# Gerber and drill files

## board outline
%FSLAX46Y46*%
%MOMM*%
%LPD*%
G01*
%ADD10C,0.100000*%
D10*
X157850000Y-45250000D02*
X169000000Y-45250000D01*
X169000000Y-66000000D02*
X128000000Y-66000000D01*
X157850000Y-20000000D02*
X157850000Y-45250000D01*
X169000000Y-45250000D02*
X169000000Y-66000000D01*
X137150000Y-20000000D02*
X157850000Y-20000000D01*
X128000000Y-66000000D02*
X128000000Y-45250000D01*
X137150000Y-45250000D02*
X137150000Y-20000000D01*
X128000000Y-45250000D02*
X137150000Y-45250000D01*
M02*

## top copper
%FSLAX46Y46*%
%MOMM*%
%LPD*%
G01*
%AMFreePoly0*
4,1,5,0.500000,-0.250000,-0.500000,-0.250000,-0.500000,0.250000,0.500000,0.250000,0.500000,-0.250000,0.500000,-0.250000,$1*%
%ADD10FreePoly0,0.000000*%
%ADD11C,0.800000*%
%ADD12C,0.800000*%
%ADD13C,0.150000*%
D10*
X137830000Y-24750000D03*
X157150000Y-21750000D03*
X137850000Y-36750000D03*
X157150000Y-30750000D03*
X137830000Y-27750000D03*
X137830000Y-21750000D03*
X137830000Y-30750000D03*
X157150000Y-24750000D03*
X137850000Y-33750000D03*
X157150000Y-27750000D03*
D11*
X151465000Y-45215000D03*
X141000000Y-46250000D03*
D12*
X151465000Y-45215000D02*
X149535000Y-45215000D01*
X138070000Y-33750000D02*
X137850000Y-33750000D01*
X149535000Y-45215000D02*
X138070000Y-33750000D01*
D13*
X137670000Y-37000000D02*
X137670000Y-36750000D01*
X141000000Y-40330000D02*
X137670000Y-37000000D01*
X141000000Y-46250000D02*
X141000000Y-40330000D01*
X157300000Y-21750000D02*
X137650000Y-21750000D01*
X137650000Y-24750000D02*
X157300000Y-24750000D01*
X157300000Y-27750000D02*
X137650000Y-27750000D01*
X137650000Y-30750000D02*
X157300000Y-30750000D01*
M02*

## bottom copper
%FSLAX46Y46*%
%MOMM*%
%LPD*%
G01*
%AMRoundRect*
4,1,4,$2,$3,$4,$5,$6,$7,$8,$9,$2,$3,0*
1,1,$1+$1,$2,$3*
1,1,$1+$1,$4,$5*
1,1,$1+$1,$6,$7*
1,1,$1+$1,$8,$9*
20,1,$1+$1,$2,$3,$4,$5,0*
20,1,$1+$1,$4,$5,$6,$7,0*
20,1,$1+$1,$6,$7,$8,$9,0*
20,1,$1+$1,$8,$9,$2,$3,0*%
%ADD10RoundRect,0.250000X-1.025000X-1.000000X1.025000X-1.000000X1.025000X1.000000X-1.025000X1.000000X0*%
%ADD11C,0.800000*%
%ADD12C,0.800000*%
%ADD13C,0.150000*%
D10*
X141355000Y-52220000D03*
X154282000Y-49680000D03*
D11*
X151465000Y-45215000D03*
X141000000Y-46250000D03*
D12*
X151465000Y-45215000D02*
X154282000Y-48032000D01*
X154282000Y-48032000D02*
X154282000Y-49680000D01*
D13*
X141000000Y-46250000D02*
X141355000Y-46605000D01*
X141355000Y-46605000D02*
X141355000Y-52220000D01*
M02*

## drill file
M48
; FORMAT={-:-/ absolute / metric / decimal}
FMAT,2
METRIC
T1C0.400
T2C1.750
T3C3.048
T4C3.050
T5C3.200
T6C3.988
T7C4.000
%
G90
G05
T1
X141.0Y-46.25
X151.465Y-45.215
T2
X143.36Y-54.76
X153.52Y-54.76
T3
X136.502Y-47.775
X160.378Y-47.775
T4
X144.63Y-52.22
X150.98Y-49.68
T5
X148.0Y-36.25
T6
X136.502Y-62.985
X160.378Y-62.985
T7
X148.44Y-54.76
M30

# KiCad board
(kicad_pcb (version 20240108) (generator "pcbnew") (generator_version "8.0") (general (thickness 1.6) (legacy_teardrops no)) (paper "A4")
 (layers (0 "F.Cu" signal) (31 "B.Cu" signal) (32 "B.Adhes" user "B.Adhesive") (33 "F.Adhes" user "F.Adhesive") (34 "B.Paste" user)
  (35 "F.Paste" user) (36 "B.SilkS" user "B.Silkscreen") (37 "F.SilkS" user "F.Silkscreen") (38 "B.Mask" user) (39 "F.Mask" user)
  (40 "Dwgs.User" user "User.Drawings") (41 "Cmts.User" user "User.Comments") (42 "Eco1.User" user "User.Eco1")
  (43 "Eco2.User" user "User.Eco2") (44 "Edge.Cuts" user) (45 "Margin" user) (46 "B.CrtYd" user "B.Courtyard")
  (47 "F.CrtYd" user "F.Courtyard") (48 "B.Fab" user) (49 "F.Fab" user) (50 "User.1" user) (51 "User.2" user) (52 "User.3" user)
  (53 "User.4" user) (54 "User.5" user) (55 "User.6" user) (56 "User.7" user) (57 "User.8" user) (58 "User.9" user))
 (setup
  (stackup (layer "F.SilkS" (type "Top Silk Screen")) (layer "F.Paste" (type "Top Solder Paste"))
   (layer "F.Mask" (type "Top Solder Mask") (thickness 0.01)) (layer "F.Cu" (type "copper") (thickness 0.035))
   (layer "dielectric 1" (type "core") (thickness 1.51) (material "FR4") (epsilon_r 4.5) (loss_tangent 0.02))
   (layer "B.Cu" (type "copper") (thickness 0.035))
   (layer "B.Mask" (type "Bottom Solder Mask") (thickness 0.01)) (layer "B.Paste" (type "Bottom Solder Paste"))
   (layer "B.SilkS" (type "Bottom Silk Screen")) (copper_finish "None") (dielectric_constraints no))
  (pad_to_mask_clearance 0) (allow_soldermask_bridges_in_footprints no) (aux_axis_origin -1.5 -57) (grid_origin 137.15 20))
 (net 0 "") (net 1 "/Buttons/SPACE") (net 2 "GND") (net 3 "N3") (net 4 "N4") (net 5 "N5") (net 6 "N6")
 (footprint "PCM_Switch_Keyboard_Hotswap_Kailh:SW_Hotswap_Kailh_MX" (layer "F.Cu") (at 148.44 54.76)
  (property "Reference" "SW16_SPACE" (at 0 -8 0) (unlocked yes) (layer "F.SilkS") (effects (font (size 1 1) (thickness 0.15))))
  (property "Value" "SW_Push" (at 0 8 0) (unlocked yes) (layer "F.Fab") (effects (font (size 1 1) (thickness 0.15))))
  (pad "" np_thru_hole circle (at -5.08 0) (size 1.75 1.75) (drill 1.75) (layers "*.Cu" "*.Mask"))
  (pad "" np_thru_hole circle (at -3.81 -2.54) (size 3.05 3.05) (drill 3.05) (layers "*.Cu" "*.Mask"))
  (pad "" np_thru_hole circle (at 0 0) (size 4 4) (drill 4) (layers "*.Cu" "*.Mask"))
  (pad "" np_thru_hole circle (at 2.54 -5.08) (size 3.05 3.05) (drill 3.05) (layers "*.Cu" "*.Mask"))
  (pad "" np_thru_hole circle (at 5.08 0) (size 1.75 1.75) (drill 1.75) (layers "*.Cu" "*.Mask"))
  (pad "1" smd roundrect (at -7.085 -2.54) (size 2.55 2.5) (layers "B.Cu" "B.Paste" "B.Mask") (roundrect_rratio 0.1)
   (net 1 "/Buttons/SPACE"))
  (pad "2" smd roundrect (at 5.842 -5.08) (size 2.55 2.5) (layers "B.Cu" "B.Paste" "B.Mask") (roundrect_rratio 0.1) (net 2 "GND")))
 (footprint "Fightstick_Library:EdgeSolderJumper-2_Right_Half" (layer "F.Cu") (at 137.18 24.75)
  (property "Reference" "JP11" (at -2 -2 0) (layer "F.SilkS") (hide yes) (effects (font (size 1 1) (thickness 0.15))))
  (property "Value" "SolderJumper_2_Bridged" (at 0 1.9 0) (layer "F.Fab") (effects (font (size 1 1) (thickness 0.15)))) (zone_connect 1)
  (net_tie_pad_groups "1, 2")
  (pad "2" smd custom (at 0.65 0) (size 1 0.5) (layers "F.Cu" "F.Mask") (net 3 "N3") (zone_connect 2) (thermal_bridge_angle 45)
   (options (clearance outline) (anchor rect)) (primitives)))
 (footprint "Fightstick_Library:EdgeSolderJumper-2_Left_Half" (layer "F.Cu") (at 157.8 21.75)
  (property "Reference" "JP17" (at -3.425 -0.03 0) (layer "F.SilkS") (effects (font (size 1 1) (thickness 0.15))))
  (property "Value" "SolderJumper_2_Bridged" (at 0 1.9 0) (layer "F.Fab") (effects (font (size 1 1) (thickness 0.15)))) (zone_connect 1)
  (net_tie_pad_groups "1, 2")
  (pad "1" smd custom (at -0.65 0) (size 1 0.5) (layers "F.Cu" "F.Mask") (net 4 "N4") (zone_connect 2) (thermal_bridge_angle 45)
   (options (clearance outline) (anchor rect)) (primitives)))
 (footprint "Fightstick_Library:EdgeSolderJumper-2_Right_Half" (layer "F.Cu") (at 137.2 36.75)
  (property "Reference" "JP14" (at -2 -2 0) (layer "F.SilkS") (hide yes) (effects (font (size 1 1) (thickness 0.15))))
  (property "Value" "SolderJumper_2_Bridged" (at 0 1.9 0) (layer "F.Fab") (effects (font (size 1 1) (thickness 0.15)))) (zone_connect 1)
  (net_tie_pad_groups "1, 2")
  (pad "2" smd custom (at 0.65 0) (size 1 0.5) (layers "F.Cu" "F.Mask") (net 1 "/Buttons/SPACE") (zone_connect 2) (thermal_bridge_angle 45)
   (options (clearance outline) (anchor rect)) (primitives)))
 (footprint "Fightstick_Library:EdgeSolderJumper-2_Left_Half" (layer "F.Cu") (at 157.8 30.75)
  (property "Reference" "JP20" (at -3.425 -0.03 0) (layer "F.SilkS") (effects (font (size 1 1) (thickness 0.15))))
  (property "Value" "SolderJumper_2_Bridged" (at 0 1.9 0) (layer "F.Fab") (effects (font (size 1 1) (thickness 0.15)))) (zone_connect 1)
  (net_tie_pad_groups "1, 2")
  (pad "1" smd custom (at -0.65 0) (size 1 0.5) (layers "F.Cu" "F.Mask") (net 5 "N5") (zone_connect 2) (thermal_bridge_angle 45)
   (options (clearance outline) (anchor rect)) (primitives)))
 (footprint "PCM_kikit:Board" (layer "F.Cu") (at 128 56.75)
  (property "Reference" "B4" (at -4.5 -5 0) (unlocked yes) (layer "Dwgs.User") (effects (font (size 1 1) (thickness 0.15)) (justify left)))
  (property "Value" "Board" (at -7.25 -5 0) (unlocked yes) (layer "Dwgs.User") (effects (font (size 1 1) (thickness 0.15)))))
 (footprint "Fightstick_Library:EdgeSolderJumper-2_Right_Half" (layer "F.Cu") (at 137.18 27.75)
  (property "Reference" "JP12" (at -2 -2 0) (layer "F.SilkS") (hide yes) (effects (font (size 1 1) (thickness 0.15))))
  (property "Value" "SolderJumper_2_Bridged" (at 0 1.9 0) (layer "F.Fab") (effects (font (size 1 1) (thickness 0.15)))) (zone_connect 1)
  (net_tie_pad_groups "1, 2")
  (pad "2" smd custom (at 0.65 0) (size 1 0.5) (layers "F.Cu" "F.Mask") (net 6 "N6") (zone_connect 2) (thermal_bridge_angle 45)
   (options (clearance outline) (anchor rect)) (primitives)))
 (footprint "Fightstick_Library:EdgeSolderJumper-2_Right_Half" (layer "F.Cu") (at 137.18 21.75)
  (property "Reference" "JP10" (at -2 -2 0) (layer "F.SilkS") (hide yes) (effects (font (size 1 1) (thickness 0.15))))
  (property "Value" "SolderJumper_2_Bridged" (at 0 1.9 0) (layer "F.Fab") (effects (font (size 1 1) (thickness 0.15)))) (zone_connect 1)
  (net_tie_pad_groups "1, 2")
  (pad "2" smd custom (at 0.65 0) (size 1 0.5) (layers "F.Cu" "F.Mask") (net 4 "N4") (zone_connect 2) (thermal_bridge_angle 45)
   (options (clearance outline) (anchor rect)) (primitives)))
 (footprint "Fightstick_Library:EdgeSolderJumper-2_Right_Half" (layer "F.Cu") (at 137.18 30.75)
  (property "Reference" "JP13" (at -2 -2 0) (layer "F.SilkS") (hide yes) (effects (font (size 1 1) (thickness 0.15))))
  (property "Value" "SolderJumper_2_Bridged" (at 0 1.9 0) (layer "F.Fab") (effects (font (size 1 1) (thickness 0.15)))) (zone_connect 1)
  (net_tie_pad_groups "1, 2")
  (pad "2" smd custom (at 0.65 0) (size 1 0.5) (layers "F.Cu" "F.Mask") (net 5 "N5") (zone_connect 2) (thermal_bridge_angle 45)
   (options (clearance outline) (anchor rect)) (primitives)))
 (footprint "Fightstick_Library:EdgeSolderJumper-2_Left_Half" (layer "F.Cu") (at 157.8 24.75)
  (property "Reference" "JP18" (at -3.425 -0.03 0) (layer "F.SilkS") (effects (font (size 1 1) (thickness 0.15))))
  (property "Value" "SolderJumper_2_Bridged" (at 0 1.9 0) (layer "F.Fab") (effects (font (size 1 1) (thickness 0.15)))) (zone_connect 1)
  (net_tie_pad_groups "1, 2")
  (pad "1" smd custom (at -0.65 0) (size 1 0.5) (layers "F.Cu" "F.Mask") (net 3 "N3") (zone_connect 2) (thermal_bridge_angle 45)
   (options (clearance outline) (anchor rect)) (primitives)))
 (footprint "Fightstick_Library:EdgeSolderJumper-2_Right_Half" (layer "F.Cu") (at 137.2 33.75)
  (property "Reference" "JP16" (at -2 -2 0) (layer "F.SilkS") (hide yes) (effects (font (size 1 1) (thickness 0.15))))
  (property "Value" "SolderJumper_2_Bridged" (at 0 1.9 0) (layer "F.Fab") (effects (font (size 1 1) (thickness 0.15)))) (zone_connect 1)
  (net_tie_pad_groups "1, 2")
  (pad "2" smd custom (at 0.65 0) (size 1 0.5) (layers "F.Cu" "F.Mask") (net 2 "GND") (zone_connect 2) (thermal_bridge_angle 45)
   (options (clearance outline) (anchor rect)) (primitives)))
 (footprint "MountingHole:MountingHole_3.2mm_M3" (layer "F.Cu") (at 148 36.25)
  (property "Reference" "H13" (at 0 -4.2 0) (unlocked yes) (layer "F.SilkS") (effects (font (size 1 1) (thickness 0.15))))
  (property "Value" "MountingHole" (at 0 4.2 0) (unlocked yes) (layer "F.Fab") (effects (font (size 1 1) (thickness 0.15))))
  (pad "" np_thru_hole circle (at 0 0) (size 3.2 3.2) (drill 3.2) (layers "*.Cu" "*.Mask")))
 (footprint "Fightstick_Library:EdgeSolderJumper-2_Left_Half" (layer "F.Cu") (at 157.8 27.75)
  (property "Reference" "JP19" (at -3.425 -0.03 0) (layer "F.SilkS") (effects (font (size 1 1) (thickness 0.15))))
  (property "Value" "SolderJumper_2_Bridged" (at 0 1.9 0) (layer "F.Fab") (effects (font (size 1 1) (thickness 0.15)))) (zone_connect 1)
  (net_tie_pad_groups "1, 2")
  (pad "1" smd custom (at -0.65 0) (size 1 0.5) (layers "F.Cu" "F.Mask") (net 6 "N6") (zone_connect 2) (thermal_bridge_angle 45)
   (options (clearance outline) (anchor rect)) (primitives)))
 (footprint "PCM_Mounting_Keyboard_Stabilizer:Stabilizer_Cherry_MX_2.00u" (layer "F.Cu") (at 148.44 54.76)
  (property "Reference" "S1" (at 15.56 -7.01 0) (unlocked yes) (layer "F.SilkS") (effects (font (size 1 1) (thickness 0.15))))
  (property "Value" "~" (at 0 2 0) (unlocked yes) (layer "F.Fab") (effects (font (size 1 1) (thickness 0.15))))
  (pad "" np_thru_hole circle (at -11.938 -6.985) (size 3.048 3.048) (drill 3.048) (layers "*.Cu" "*.Mask"))
  (pad "" np_thru_hole circle (at -11.938 8.225) (size 3.9878 3.9878) (drill 3.9878) (layers "*.Cu" "*.Mask"))
  (pad "" np_thru_hole circle (at 11.938 -6.985) (size 3.048 3.048) (drill 3.048) (layers "*.Cu" "*.Mask"))
  (pad "" np_thru_hole circle (at 11.938 8.225) (size 3.9878 3.9878) (drill 3.9878) (layers "*.Cu" "*.Mask")))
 (gr_line (start 157.85 45.25) (end 169 45.25) (stroke (width 0.1) (type default)) (layer "Edge.Cuts"))
 (gr_line (start 169 66) (end 128 66) (stroke (width 0.1) (type default)) (layer "Edge.Cuts"))
 (gr_line (start 157.85 20) (end 157.85 45.25) (stroke (width 0.1) (type default)) (layer "Edge.Cuts"))
 (gr_line (start 169 45.25) (end 169 66) (stroke (width 0.1) (type default)) (layer "Edge.Cuts"))
 (gr_line (start 137.15 20) (end 157.85 20) (stroke (width 0.1) (type default)) (layer "Edge.Cuts"))
 (gr_line (start 128 66) (end 128 45.25) (stroke (width 0.1) (type default)) (layer "Edge.Cuts"))
 (gr_line (start 137.15 45.25) (end 137.15 20) (stroke (width 0.1) (type default)) (layer "Edge.Cuts"))
 (gr_line (start 128 45.25) (end 137.15 45.25) (stroke (width 0.1) (type default)) (layer "Edge.Cuts"))
 (segment (start 151.465 45.215) (end 149.535 45.215) (width 0.8) (layer "F.Cu") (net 2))
 (segment (start 138.07 33.75) (end 137.85 33.75) (width 0.8) (layer "F.Cu") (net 2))
 (segment (start 149.535 45.215) (end 138.07 33.75) (width 0.8) (layer "F.Cu") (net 2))
 (via (at 151.465 45.215) (size 0.8) (drill 0.4) (layers "F.Cu" "B.Cu") (free yes) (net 2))
 (segment (start 151.465 45.215) (end 154.282 48.032) (width 0.8) (layer "B.Cu") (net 2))
 (segment (start 154.282 48.032) (end 154.282 49.68) (width 0.8) (layer "B.Cu") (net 2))
 (segment (start 137.67 37) (end 137.67 36.75) (width 0.15) (layer "F.Cu") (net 1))
 (segment (start 141 40.33) (end 137.67 37) (width 0.15) (layer "F.Cu") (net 1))
 (segment (start 141 46.25) (end 141 40.33) (width 0.15) (layer "F.Cu") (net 1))
 (via (at 141 46.25) (size 0.8) (drill 0.4) (layers "F.Cu" "B.Cu") (free yes) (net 1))
 (segment (start 141 46.25) (end 141.355 46.605) (width 0.15) (layer "B.Cu") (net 1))
 (segment (start 141.355 46.605) (end 141.355 52.22) (width 0.15) (layer "B.Cu") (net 1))
 (segment (start 157.3 21.75) (end 137.65 21.75) (width 0.15) (layer "F.Cu") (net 4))
 (segment (start 137.65 24.75) (end 157.3 24.75) (width 0.15) (layer "F.Cu") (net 3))
 (segment (start 157.3 27.75) (end 137.65 27.75) (width 0.15) (layer "F.Cu") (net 6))
 (segment (start 137.65 30.75) (end 157.3 30.75) (width 0.15) (layer "F.Cu") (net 5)))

